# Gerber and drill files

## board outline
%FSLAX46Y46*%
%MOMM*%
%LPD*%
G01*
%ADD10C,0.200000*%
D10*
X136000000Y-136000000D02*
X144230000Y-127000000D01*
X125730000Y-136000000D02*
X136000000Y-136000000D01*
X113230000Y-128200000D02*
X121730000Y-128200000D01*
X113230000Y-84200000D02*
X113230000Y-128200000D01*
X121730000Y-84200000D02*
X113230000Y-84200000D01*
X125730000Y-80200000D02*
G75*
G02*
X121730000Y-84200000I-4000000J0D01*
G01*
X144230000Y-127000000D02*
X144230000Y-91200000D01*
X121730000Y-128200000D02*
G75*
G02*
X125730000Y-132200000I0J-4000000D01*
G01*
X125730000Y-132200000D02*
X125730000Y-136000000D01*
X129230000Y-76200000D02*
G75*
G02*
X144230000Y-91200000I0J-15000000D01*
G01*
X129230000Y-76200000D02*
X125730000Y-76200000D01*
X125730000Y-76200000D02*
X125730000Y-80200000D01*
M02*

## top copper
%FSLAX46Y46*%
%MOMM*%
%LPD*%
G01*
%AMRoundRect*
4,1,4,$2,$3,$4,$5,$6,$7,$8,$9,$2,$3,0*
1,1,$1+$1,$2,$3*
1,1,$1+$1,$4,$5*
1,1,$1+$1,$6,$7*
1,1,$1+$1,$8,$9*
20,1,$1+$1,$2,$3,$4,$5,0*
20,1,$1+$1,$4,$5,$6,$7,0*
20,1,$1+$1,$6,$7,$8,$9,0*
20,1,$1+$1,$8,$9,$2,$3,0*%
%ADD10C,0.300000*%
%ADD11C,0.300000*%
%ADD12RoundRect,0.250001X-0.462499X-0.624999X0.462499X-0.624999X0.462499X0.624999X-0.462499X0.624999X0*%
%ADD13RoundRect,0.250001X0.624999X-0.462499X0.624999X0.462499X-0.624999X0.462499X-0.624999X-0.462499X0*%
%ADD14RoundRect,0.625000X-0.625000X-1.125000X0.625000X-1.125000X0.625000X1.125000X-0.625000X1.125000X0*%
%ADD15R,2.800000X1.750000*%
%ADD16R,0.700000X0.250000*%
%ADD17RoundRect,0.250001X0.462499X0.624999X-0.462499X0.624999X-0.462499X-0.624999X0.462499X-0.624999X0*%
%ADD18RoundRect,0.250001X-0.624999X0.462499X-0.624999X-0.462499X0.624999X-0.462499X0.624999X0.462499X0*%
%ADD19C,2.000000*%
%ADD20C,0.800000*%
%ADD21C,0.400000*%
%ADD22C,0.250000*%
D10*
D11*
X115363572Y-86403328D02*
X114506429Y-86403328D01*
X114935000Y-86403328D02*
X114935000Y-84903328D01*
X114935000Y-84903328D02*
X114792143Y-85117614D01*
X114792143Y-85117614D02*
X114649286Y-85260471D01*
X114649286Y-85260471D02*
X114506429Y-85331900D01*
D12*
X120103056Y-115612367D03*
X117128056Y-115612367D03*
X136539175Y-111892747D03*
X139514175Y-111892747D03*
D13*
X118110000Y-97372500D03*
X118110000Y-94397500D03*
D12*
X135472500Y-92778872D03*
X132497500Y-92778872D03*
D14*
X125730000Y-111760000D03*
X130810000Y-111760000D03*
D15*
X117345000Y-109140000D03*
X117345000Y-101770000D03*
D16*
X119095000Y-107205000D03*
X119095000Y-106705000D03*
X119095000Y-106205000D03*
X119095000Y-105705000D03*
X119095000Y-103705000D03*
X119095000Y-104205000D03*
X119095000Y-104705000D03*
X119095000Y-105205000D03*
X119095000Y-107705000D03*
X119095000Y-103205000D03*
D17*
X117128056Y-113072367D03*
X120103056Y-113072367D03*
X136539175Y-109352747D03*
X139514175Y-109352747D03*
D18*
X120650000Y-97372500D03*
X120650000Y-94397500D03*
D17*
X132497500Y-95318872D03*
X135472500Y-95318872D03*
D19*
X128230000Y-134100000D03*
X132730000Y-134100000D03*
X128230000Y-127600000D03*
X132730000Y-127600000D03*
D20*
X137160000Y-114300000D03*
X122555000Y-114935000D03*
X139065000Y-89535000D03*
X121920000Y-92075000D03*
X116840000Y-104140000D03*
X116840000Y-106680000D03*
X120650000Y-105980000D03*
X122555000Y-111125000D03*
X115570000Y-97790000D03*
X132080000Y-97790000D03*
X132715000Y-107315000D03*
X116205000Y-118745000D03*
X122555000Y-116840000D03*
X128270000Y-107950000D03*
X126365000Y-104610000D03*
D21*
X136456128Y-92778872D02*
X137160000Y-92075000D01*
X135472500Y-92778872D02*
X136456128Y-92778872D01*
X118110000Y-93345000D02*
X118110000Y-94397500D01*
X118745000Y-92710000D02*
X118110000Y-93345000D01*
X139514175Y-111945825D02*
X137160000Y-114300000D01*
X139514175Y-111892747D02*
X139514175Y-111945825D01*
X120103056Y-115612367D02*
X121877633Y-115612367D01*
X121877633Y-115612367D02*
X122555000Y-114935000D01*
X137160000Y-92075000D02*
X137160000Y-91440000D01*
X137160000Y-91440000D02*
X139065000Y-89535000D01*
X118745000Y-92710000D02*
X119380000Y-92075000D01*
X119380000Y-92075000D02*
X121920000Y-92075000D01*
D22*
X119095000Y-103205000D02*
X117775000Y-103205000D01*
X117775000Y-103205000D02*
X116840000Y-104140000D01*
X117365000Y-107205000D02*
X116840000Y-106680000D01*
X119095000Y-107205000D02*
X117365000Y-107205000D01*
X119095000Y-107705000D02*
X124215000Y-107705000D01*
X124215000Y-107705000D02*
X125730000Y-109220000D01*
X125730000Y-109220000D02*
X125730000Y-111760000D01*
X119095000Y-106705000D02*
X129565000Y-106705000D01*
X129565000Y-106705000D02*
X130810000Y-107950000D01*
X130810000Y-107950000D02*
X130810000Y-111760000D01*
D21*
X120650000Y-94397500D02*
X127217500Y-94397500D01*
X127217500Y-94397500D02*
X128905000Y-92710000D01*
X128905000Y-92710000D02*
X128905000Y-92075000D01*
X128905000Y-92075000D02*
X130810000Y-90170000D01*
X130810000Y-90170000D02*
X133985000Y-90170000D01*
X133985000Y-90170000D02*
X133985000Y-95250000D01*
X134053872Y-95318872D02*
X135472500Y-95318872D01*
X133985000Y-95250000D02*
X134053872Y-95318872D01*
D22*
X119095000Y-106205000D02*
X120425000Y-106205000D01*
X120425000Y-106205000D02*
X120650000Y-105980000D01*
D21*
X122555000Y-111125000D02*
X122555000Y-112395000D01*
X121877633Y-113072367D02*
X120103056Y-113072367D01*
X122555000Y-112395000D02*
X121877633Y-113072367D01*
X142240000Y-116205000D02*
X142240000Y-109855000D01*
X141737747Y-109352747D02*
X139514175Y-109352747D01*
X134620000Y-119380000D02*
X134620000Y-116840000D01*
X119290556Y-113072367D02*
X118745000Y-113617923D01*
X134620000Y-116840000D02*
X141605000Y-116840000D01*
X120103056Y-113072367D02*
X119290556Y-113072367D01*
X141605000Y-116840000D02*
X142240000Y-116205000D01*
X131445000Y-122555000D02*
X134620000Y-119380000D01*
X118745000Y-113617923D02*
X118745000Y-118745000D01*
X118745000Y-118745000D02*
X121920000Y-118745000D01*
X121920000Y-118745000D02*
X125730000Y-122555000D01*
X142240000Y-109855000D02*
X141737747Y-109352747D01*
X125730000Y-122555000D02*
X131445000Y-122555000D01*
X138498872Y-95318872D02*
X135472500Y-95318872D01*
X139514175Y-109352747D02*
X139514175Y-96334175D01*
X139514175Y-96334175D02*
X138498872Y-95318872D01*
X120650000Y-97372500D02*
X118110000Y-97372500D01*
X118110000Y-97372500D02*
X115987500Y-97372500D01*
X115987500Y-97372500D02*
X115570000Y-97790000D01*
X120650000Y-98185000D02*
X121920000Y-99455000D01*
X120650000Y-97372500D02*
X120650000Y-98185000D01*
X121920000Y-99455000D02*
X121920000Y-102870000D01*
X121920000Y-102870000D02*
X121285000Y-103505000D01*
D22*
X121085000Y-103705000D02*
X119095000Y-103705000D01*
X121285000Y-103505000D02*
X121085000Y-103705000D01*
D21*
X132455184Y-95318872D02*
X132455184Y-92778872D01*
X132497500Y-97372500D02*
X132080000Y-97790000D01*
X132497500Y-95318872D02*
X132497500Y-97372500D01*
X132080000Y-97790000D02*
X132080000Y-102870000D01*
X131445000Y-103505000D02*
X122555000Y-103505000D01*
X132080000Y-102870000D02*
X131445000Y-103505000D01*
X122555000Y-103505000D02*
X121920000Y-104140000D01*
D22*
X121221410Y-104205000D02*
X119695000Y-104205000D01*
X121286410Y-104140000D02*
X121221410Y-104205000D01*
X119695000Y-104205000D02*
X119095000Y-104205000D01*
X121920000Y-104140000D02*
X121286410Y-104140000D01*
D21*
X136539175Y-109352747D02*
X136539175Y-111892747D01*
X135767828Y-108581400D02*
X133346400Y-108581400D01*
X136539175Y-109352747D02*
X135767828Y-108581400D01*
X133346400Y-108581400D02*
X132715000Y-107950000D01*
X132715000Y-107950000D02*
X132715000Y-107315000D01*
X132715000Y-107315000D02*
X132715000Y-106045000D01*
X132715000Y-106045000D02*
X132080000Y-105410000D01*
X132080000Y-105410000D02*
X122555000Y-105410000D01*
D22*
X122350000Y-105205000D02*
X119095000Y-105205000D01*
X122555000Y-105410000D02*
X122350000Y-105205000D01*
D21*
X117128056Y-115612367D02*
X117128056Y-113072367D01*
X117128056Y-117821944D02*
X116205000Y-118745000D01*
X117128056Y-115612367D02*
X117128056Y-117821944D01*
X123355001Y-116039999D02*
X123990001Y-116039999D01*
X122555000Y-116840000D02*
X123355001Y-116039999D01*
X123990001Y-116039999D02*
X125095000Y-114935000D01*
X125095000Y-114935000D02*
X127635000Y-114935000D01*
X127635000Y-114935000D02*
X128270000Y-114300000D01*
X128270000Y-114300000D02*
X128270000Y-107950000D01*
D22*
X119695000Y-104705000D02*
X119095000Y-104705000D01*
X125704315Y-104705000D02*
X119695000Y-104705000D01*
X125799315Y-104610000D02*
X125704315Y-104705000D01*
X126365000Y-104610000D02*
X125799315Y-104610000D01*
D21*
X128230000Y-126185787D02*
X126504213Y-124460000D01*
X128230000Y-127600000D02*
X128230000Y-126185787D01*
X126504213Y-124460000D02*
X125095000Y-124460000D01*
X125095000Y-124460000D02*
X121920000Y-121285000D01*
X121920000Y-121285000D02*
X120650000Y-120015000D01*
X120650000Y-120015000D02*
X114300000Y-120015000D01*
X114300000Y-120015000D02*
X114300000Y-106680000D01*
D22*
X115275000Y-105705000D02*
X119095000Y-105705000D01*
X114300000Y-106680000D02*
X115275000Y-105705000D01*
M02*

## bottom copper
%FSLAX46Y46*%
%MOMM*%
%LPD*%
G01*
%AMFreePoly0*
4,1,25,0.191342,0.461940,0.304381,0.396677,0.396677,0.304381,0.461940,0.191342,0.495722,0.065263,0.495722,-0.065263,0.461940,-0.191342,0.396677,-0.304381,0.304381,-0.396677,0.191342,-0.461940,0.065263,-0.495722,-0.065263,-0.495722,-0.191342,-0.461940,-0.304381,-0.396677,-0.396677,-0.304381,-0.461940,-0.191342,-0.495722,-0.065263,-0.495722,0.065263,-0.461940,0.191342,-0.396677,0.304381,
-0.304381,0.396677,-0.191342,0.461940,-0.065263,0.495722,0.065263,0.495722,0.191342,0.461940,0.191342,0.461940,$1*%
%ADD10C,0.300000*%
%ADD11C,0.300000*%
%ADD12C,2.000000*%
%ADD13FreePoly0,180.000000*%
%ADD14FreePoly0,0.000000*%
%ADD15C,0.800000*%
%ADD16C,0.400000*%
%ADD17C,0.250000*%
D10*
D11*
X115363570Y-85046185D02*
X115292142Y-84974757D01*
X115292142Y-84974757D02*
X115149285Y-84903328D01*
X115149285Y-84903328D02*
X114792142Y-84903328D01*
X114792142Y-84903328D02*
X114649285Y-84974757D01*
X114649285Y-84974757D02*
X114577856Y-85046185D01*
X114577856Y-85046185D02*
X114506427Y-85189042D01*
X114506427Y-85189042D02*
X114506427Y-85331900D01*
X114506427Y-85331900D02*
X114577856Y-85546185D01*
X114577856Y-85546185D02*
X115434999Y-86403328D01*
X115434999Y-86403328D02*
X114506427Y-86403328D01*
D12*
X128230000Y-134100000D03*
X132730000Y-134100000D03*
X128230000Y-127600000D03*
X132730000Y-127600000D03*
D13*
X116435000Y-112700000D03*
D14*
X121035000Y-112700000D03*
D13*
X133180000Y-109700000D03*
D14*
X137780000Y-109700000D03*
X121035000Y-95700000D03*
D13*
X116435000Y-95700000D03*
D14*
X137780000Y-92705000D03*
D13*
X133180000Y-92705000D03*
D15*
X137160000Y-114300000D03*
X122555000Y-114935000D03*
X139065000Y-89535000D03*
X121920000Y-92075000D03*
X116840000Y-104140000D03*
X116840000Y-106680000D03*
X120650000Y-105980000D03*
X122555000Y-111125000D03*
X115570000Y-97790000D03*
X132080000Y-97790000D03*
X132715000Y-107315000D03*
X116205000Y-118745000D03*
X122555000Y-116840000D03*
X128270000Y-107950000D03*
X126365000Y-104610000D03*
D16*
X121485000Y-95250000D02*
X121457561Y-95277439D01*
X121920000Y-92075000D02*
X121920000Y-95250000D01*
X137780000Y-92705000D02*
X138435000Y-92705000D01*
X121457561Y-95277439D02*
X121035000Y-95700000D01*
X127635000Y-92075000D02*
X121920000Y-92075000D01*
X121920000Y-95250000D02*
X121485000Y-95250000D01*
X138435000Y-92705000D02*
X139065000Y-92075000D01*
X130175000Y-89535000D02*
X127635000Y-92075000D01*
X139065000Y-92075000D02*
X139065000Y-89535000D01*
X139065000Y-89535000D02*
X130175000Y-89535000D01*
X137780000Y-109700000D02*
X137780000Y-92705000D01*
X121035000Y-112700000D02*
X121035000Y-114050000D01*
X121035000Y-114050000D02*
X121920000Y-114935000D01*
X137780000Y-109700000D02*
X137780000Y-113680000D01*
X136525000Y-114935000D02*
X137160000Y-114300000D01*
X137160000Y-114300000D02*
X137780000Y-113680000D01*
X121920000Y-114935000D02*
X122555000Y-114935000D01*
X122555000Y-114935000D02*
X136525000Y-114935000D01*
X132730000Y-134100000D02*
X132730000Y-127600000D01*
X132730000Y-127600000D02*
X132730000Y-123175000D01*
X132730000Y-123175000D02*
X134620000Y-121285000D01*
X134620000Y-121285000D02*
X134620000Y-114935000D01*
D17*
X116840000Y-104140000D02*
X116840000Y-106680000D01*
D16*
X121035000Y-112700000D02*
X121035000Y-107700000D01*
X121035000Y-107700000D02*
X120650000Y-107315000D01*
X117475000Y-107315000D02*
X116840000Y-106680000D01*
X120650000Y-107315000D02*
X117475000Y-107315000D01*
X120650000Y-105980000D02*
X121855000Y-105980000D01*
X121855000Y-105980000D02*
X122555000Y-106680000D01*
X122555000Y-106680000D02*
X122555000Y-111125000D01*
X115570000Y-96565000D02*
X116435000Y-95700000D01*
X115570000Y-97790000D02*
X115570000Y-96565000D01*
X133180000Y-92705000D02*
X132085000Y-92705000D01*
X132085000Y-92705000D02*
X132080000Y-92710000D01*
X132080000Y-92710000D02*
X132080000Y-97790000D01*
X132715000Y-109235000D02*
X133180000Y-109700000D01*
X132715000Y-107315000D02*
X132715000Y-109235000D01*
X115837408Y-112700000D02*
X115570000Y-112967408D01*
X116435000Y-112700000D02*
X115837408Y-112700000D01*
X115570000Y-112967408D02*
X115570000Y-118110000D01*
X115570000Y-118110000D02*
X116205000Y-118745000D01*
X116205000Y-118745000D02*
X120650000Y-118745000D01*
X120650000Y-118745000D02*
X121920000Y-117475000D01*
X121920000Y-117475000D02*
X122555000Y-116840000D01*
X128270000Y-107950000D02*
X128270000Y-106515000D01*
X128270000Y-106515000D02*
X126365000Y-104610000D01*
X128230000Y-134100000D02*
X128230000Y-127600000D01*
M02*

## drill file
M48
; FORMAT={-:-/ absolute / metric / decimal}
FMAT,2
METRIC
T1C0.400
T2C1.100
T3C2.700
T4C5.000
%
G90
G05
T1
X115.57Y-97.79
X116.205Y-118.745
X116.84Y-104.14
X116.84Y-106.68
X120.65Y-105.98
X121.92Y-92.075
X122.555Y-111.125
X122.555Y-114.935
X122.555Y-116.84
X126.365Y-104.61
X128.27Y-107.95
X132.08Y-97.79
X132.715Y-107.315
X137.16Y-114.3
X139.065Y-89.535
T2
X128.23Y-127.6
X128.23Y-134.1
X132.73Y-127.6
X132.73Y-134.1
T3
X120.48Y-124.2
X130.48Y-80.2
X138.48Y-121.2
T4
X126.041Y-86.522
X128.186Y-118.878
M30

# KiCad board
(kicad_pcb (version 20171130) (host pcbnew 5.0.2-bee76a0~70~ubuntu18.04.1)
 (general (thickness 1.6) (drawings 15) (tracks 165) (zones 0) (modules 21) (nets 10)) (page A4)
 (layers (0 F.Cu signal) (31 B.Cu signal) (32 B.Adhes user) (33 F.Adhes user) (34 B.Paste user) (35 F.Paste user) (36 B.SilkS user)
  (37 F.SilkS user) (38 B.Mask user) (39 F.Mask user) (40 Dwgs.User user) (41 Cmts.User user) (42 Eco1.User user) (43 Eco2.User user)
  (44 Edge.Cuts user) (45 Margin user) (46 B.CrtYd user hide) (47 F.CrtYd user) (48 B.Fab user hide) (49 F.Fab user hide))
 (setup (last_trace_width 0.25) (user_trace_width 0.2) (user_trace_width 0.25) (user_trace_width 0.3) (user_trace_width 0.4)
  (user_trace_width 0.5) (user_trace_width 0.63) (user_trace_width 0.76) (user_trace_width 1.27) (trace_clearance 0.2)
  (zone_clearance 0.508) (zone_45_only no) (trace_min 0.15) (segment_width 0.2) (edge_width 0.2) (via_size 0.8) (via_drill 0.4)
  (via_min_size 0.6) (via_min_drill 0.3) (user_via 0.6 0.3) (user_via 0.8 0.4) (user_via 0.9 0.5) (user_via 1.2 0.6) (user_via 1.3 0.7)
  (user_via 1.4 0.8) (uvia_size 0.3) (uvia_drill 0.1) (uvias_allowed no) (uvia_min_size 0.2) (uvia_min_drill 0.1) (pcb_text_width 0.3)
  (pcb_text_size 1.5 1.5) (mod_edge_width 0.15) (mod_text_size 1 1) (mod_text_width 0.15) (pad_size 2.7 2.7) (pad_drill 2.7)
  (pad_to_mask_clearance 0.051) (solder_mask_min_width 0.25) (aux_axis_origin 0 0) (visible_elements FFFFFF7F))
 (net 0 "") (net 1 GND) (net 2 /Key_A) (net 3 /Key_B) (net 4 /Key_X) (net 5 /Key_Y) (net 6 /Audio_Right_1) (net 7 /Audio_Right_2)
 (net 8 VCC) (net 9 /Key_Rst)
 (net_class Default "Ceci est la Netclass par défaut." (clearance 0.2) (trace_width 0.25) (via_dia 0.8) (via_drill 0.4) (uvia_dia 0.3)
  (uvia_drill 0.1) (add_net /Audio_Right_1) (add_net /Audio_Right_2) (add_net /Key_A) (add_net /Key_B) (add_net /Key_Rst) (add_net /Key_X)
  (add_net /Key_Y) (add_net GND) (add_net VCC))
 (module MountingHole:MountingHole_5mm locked (layer F.Cu) (at 126.041 86.522)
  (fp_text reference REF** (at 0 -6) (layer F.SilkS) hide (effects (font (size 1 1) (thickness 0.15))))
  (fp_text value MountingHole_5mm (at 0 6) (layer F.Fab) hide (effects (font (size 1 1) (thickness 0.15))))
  (pad "" np_thru_hole circle (at 0 0) (size 5 5) (drill 5) (layers *.Cu *.Mask)))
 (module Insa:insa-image (layer F.Cu) (at 130.81 101.6)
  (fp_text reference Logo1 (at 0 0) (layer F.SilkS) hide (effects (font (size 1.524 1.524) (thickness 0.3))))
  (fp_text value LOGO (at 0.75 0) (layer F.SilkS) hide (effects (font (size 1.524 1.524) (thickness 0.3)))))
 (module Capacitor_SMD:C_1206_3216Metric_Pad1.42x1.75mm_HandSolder (layer F.Cu) (at 118.615556 115.612367)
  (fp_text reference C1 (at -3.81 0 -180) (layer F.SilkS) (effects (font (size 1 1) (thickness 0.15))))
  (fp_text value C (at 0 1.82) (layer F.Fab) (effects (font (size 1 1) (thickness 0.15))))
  (pad 2 smd roundrect (at 1.4875 0) (size 1.425 1.75) (layers F.Cu F.Paste F.Mask) (roundrect_rratio 0.175439) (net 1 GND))
  (pad 1 smd roundrect (at -1.4875 0) (size 1.425 1.75) (layers F.Cu F.Paste F.Mask) (roundrect_rratio 0.175439) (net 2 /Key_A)))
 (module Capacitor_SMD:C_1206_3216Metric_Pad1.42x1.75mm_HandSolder (layer F.Cu) (at 138.026675 111.892747)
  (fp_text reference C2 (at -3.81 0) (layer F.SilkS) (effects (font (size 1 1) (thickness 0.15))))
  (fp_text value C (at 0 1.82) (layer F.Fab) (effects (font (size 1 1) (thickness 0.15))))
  (pad 1 smd roundrect (at -1.4875 0) (size 1.425 1.75) (layers F.Cu F.Paste F.Mask) (roundrect_rratio 0.175439) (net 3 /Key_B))
  (pad 2 smd roundrect (at 1.4875 0) (size 1.425 1.75) (layers F.Cu F.Paste F.Mask) (roundrect_rratio 0.175439) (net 1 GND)))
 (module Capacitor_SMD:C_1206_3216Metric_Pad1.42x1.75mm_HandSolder (layer F.Cu) (at 118.11 95.885 90)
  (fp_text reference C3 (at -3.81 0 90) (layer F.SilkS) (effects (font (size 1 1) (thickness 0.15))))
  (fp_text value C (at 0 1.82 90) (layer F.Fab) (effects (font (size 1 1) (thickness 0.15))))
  (pad 1 smd roundrect (at -1.4875 0 90) (size 1.425 1.75) (layers F.Cu F.Paste F.Mask) (roundrect_rratio 0.175439) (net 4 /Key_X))
  (pad 2 smd roundrect (at 1.4875 0 90) (size 1.425 1.75) (layers F.Cu F.Paste F.Mask) (roundrect_rratio 0.175439) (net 1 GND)))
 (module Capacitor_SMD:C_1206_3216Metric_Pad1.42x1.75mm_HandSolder (layer F.Cu) (at 133.985 92.778872)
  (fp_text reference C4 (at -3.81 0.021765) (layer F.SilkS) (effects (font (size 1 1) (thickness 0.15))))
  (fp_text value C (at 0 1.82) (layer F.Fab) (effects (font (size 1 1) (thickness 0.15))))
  (pad 2 smd roundrect (at 1.4875 0) (size 1.425 1.75) (layers F.Cu F.Paste F.Mask) (roundrect_rratio 0.175439) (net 1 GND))
  (pad 1 smd roundrect (at -1.4875 0) (size 1.425 1.75) (layers F.Cu F.Paste F.Mask) (roundrect_rratio 0.175439) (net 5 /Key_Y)))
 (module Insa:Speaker (layer F.Cu) (at 128.27 111.76)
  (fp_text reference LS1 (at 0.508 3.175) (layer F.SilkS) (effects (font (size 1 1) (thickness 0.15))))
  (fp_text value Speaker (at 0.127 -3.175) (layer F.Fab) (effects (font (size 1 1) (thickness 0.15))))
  (pad 1 smd roundrect (at -2.54 0) (size 2.5 3.5) (layers F.Cu F.Paste F.Mask) (roundrect_rratio 0.25) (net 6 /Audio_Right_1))
  (pad 2 smd roundrect (at 2.54 0) (size 2.5 3.5) (layers F.Cu F.Paste F.Mask) (roundrect_rratio 0.25) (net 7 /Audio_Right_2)))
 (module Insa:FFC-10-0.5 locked (layer F.Cu) (at 118.745 105.455 90)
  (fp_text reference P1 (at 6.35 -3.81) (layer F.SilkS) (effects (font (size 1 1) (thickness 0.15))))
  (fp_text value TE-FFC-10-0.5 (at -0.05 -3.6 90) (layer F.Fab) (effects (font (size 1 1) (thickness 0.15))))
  (pad A smd rect (at -3.685 -1.4 90) (size 1.75 2.8) (layers F.Cu F.Paste F.Mask))
  (pad B smd rect (at 3.685 -1.4 90) (size 1.75 2.8) (layers F.Cu F.Paste F.Mask))
  (pad 2 smd rect (at -1.75 0.35 90) (size 0.25 0.7) (layers F.Cu F.Paste F.Mask) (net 1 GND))
  (pad 3 smd rect (at -1.25 0.35 90) (size 0.25 0.7) (layers F.Cu F.Paste F.Mask) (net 7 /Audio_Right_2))
  (pad 4 smd rect (at -0.75 0.35 90) (size 0.25 0.7) (layers F.Cu F.Paste F.Mask) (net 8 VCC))
  (pad 5 smd rect (at -0.25 0.35 90) (size 0.25 0.7) (layers F.Cu F.Paste F.Mask) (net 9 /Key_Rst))
  (pad 9 smd rect (at 1.75 0.35 90) (size 0.25 0.7) (layers F.Cu F.Paste F.Mask) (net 4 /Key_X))
  (pad 8 smd rect (at 1.25 0.35 90) (size 0.25 0.7) (layers F.Cu F.Paste F.Mask) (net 5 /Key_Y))
  (pad 7 smd rect (at 0.75 0.35 90) (size 0.25 0.7) (layers F.Cu F.Paste F.Mask) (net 2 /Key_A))
  (pad 6 smd rect (at 0.25 0.35 90) (size 0.25 0.7) (layers F.Cu F.Paste F.Mask) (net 3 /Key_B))
  (pad 1 smd rect (at -2.25 0.35 90) (size 0.25 0.7) (layers F.Cu F.Paste F.Mask) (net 6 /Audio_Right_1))
  (pad 10 smd rect (at 2.25 0.35 90) (size 0.25 0.7) (layers F.Cu F.Paste F.Mask) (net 1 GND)))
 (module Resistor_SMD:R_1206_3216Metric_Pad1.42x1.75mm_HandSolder (layer F.Cu) (at 118.615556 113.072367 180)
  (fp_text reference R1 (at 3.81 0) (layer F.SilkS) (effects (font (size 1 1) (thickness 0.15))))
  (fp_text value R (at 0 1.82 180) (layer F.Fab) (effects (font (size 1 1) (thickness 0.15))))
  (pad 2 smd roundrect (at 1.4875 0 180) (size 1.425 1.75) (layers F.Cu F.Paste F.Mask) (roundrect_rratio 0.175439) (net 2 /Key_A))
  (pad 1 smd roundrect (at -1.4875 0 180) (size 1.425 1.75) (layers F.Cu F.Paste F.Mask) (roundrect_rratio 0.175439) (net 8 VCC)))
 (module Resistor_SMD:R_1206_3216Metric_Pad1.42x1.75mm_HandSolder (layer F.Cu) (at 138.026675 109.352747 180)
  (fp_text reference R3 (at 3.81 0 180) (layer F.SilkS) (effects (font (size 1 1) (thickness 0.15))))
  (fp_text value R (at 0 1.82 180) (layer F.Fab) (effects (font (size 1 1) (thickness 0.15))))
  (pad 2 smd roundrect (at 1.4875 0 180) (size 1.425 1.75) (layers F.Cu F.Paste F.Mask) (roundrect_rratio 0.175439) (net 3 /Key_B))
  (pad 1 smd roundrect (at -1.4875 0 180) (size 1.425 1.75) (layers F.Cu F.Paste F.Mask) (roundrect_rratio 0.175439) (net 8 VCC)))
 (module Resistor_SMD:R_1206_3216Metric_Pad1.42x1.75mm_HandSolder (layer F.Cu) (at 120.65 95.885 270)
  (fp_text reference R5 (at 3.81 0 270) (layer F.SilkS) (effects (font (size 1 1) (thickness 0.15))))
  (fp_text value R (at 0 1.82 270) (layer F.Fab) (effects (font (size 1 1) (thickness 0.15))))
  (pad 2 smd roundrect (at 1.4875 0 270) (size 1.425 1.75) (layers F.Cu F.Paste F.Mask) (roundrect_rratio 0.175439) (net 4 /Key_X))
  (pad 1 smd roundrect (at -1.4875 0 270) (size 1.425 1.75) (layers F.Cu F.Paste F.Mask) (roundrect_rratio 0.175439) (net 8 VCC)))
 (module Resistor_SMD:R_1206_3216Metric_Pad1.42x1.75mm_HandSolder (layer F.Cu) (at 133.985 95.318872 180)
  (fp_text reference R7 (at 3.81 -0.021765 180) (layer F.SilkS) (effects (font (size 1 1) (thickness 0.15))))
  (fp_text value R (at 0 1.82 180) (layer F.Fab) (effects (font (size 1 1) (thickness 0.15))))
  (pad 2 smd roundrect (at 1.4875 0 180) (size 1.425 1.75) (layers F.Cu F.Paste F.Mask) (roundrect_rratio 0.175439) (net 5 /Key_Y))
  (pad 1 smd roundrect (at -1.4875 0 180) (size 1.425 1.75) (layers F.Cu F.Paste F.Mask) (roundrect_rratio 0.175439) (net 8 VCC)))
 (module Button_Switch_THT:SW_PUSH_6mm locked (layer B.Cu) (at 132.73 134.1 90)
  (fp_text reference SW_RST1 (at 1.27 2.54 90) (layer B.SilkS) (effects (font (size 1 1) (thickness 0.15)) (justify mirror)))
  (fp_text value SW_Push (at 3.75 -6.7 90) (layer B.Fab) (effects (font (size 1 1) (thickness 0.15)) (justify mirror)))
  (pad 2 thru_hole circle (at 0 -4.5) (size 2 2) (drill 1.1) (layers *.Cu *.Mask) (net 9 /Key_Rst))
  (pad 1 thru_hole circle (at 0 0) (size 2 2) (drill 1.1) (layers *.Cu *.Mask) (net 1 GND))
  (pad 2 thru_hole circle (at 6.5 -4.5) (size 2 2) (drill 1.1) (layers *.Cu *.Mask) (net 9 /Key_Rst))
  (pad 1 thru_hole circle (at 6.5 0) (size 2 2) (drill 1.1) (layers *.Cu *.Mask) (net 1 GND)))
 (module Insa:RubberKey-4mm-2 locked (layer B.Cu) (at 118.735 112.7)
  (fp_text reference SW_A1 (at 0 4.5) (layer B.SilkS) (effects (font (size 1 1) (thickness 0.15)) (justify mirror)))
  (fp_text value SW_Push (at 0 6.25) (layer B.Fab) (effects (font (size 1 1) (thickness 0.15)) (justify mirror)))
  (pad 2 smd custom (at -2.3 0 180) (size 1 1) (layers B.Cu B.Paste B.Mask) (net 2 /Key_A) (zone_connect 0)
   (options (clearance outline) (anchor circle)) (primitives))
  (pad 1 smd custom (at 2.3 0) (size 1 1) (layers B.Cu B.Paste B.Mask) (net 1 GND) (zone_connect 0)
   (options (clearance outline) (anchor circle)) (primitives)))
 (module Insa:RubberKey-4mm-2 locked (layer B.Cu) (at 135.48 109.7)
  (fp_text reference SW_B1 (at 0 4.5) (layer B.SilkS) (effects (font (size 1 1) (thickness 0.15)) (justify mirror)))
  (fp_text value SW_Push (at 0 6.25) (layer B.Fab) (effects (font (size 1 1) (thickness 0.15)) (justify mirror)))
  (pad 2 smd custom (at -2.3 0 180) (size 1 1) (layers B.Cu B.Paste B.Mask) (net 3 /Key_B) (zone_connect 0)
   (options (clearance outline) (anchor circle)) (primitives))
  (pad 1 smd custom (at 2.3 0) (size 1 1) (layers B.Cu B.Paste B.Mask) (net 1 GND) (zone_connect 0)
   (options (clearance outline) (anchor circle)) (primitives)))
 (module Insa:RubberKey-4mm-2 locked (layer B.Cu) (at 118.735 95.7)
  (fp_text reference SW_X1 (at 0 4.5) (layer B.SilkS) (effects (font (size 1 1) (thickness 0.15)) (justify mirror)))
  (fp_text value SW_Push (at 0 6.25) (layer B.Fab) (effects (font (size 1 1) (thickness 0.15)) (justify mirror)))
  (pad 1 smd custom (at 2.3 0) (size 1 1) (layers B.Cu B.Paste B.Mask) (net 1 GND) (zone_connect 0)
   (options (clearance outline) (anchor circle)) (primitives))
  (pad 2 smd custom (at -2.3 0 180) (size 1 1) (layers B.Cu B.Paste B.Mask) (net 4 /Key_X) (zone_connect 0)
   (options (clearance outline) (anchor circle)) (primitives)))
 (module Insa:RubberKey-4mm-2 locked (layer B.Cu) (at 135.48 92.705)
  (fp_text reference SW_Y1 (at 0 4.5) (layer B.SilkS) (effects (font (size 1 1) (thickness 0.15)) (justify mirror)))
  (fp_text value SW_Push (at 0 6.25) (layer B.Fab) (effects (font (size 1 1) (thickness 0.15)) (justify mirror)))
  (pad 1 smd custom (at 2.3 0) (size 1 1) (layers B.Cu B.Paste B.Mask) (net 1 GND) (zone_connect 0)
   (options (clearance outline) (anchor circle)) (primitives))
  (pad 2 smd custom (at -2.3 0 180) (size 1 1) (layers B.Cu B.Paste B.Mask) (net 5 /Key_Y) (zone_connect 0)
   (options (clearance outline) (anchor circle)) (primitives)))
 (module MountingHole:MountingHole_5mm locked (layer F.Cu) (at 128.186 118.878)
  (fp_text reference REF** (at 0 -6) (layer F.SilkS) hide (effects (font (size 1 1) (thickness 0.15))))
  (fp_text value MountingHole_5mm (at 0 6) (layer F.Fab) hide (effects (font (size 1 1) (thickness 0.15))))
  (pad "" np_thru_hole circle (at 0 0) (size 5 5) (drill 5) (layers *.Cu *.Mask)))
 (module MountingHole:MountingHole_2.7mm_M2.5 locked (layer F.Cu) (at 138.48 121.2)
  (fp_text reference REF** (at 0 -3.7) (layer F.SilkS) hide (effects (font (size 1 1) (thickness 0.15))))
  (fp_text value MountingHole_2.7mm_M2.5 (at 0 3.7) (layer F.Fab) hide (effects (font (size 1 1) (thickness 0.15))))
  (pad "" np_thru_hole circle (at 0 0) (size 2.7 2.7) (drill 2.7) (layers *.Cu *.Mask)))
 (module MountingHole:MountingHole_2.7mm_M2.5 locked (layer F.Cu) (at 120.48 124.2)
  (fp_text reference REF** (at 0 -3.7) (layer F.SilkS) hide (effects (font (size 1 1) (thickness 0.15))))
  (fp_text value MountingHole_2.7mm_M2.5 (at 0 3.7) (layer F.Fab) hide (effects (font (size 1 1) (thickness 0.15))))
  (pad "" np_thru_hole circle (at 0 0) (size 2.7 2.7) (drill 2.7) (layers *.Cu *.Mask)))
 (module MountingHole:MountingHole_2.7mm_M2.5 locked (layer F.Cu) (at 130.48 80.2)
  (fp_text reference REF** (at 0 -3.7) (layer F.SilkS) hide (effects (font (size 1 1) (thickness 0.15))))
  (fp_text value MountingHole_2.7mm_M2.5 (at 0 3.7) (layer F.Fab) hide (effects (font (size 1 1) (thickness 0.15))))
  (pad "" np_thru_hole circle (at 0 0) (size 2.7 2.7) (drill 2.7) (layers *.Cu *.Mask)))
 (gr_line (start 136 136) (end 144.23 127) (layer Edge.Cuts) (width 0.2))
 (gr_line (start 125.73 136) (end 136 136) (layer Edge.Cuts) (width 0.2))
 (gr_line (start 113.23 128.2) (end 121.73 128.2) (layer Edge.Cuts) (width 0.2))
 (gr_line (start 113.23 84.2) (end 113.23 128.2) (layer Edge.Cuts) (width 0.2))
 (gr_line (start 121.73 84.2) (end 113.23 84.2) (layer Edge.Cuts) (width 0.2))
 (gr_arc (start 121.73 80.2) (end 121.73 84.2) (angle -90) (layer Edge.Cuts) (width 0.2))
 (gr_line (start 144.23 127) (end 144.23 91.2) (layer Edge.Cuts) (width 0.2))
 (gr_arc (start 121.73 132.2) (end 125.73 132.2) (angle -90) (layer Edge.Cuts) (width 0.2))
 (gr_line (start 125.73 132.2) (end 125.73 136) (layer Edge.Cuts) (width 0.2))
 (gr_arc (start 129.23 91.2) (end 144.23 91.2) (angle -90) (layer Edge.Cuts) (width 0.2))
 (gr_line (start 129.23 76.2) (end 125.73 76.2) (layer Edge.Cuts) (width 0.2))
 (gr_line (start 125.73 76.2) (end 125.73 80.2) (layer Edge.Cuts) (width 0.2))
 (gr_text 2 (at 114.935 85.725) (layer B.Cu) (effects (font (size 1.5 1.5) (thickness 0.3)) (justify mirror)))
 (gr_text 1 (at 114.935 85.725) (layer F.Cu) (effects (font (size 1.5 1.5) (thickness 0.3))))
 (segment (start 136.456128 92.778872) (end 137.16 92.075) (width 0.4) (layer F.Cu) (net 1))
 (segment (start 135.4725 92.778872) (end 136.456128 92.778872) (width 0.4) (layer F.Cu) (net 1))
 (segment (start 118.11 93.345) (end 118.11 94.3975) (width 0.4) (layer F.Cu) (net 1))
 (segment (start 118.745 92.71) (end 118.11 93.345) (width 0.4) (layer F.Cu) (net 1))
 (segment (start 121.485 95.25) (end 121.457561 95.277439) (width 0.4) (layer B.Cu) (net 1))
 (segment (start 121.92 92.075) (end 121.92 95.25) (width 0.4) (layer B.Cu) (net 1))
 (segment (start 137.78 92.705) (end 138.435 92.705) (width 0.4) (layer B.Cu) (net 1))
 (segment (start 121.457561 95.277439) (end 121.035 95.7) (width 0.4) (layer B.Cu) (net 1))
 (segment (start 127.635 92.075) (end 121.92 92.075) (width 0.4) (layer B.Cu) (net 1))
 (segment (start 121.92 95.25) (end 121.485 95.25) (width 0.4) (layer B.Cu) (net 1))
 (segment (start 138.435 92.705) (end 139.065 92.075) (width 0.4) (layer B.Cu) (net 1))
 (segment (start 130.175 89.535) (end 127.635 92.075) (width 0.4) (layer B.Cu) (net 1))
 (segment (start 139.065 92.075) (end 139.065 89.535) (width 0.4) (layer B.Cu) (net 1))
 (segment (start 139.065 89.535) (end 130.175 89.535) (width 0.4) (layer B.Cu) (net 1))
 (segment (start 137.78 109.7) (end 137.78 92.705) (width 0.4) (layer B.Cu) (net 1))
 (segment (start 121.035 112.7) (end 121.035 114.05) (width 0.4) (layer B.Cu) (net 1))
 (segment (start 121.035 114.05) (end 121.92 114.935) (width 0.4) (layer B.Cu) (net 1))
 (segment (start 137.78 109.7) (end 137.78 113.68) (width 0.4) (layer B.Cu) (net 1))
 (via (at 137.16 114.3) (size 0.8) (drill 0.4) (layers F.Cu B.Cu) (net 1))
 (segment (start 139.514175 111.945825) (end 137.16 114.3) (width 0.4) (layer F.Cu) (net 1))
 (segment (start 139.514175 111.892747) (end 139.514175 111.945825) (width 0.4) (layer F.Cu) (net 1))
 (segment (start 136.525 114.935) (end 137.16 114.3) (width 0.4) (layer B.Cu) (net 1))
 (segment (start 137.16 114.3) (end 137.78 113.68) (width 0.4) (layer B.Cu) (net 1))
 (segment (start 120.103056 115.612367) (end 121.877633 115.612367) (width 0.4) (layer F.Cu) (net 1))
 (via (at 122.555 114.935) (size 0.8) (drill 0.4) (layers F.Cu B.Cu) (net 1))
 (segment (start 121.877633 115.612367) (end 122.555 114.935) (width 0.4) (layer F.Cu) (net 1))
 (segment (start 121.92 114.935) (end 122.555 114.935) (width 0.4) (layer B.Cu) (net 1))
 (segment (start 122.555 114.935) (end 136.525 114.935) (width 0.4) (layer B.Cu) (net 1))
 (segment (start 132.73 134.1) (end 132.73 127.6) (width 0.4) (layer B.Cu) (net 1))
 (segment (start 132.73 127.6) (end 132.73 123.175) (width 0.4) (layer B.Cu) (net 1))
 (segment (start 132.73 123.175) (end 134.62 121.285) (width 0.4) (layer B.Cu) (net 1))
 (segment (start 134.62 121.285) (end 134.62 114.935) (width 0.4) (layer B.Cu) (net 1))
 (segment (start 137.16 92.075) (end 137.16 91.44) (width 0.4) (layer F.Cu) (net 1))
 (segment (start 137.16 91.44) (end 139.065 89.535) (width 0.4) (layer F.Cu) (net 1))
 (via (at 139.065 89.535) (size 0.8) (drill 0.4) (layers F.Cu B.Cu) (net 1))
 (segment (start 118.745 92.71) (end 119.38 92.075) (width 0.4) (layer F.Cu) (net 1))
 (segment (start 119.38 92.075) (end 121.92 92.075) (width 0.4) (layer F.Cu) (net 1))
 (via (at 121.92 92.075) (size 0.8) (drill 0.4) (layers F.Cu B.Cu) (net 1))
 (segment (start 119.095 103.205) (end 117.775 103.205) (width 0.25) (layer F.Cu) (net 1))
 (via (at 116.84 104.14) (size 0.8) (drill 0.4) (layers F.Cu B.Cu) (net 1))
 (segment (start 117.775 103.205) (end 116.84 104.14) (width 0.25) (layer F.Cu) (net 1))
 (segment (start 116.84 104.14) (end 116.84 106.68) (width 0.25) (layer B.Cu) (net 1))
 (via (at 116.84 106.68) (size 0.8) (drill 0.4) (layers F.Cu B.Cu) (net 1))
 (segment (start 117.365 107.205) (end 116.84 106.68) (width 0.25) (layer F.Cu) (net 1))
 (segment (start 119.095 107.205) (end 117.365 107.205) (width 0.25) (layer F.Cu) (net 1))
 (segment (start 121.035 112.7) (end 121.035 107.7) (width 0.4) (layer B.Cu) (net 1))
 (segment (start 121.035 107.7) (end 120.65 107.315) (width 0.4) (layer B.Cu) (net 1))
 (segment (start 117.475 107.315) (end 116.84 106.68) (width 0.4) (layer B.Cu) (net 1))
 (segment (start 120.65 107.315) (end 117.475 107.315) (width 0.4) (layer B.Cu) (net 1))
 (segment (start 119.095 107.705) (end 124.215 107.705) (width 0.25) (layer F.Cu) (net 6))
 (segment (start 124.215 107.705) (end 125.73 109.22) (width 0.25) (layer F.Cu) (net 6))
 (segment (start 125.73 109.22) (end 125.73 111.76) (width 0.25) (layer F.Cu) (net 6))
 (segment (start 119.095 106.705) (end 129.565 106.705) (width 0.25) (layer F.Cu) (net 7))
 (segment (start 129.565 106.705) (end 130.81 107.95) (width 0.25) (layer F.Cu) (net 7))
 (segment (start 130.81 107.95) (end 130.81 111.76) (width 0.25) (layer F.Cu) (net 7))
 (segment (start 120.65 94.3975) (end 127.2175 94.3975) (width 0.4) (layer F.Cu) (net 8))
 (segment (start 127.2175 94.3975) (end 128.905 92.71) (width 0.4) (layer F.Cu) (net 8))
 (segment (start 128.905 92.71) (end 128.905 92.075) (width 0.4) (layer F.Cu) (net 8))
 (segment (start 128.905 92.075) (end 130.81 90.17) (width 0.4) (layer F.Cu) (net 8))
 (segment (start 130.81 90.17) (end 133.985 90.17) (width 0.4) (layer F.Cu) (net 8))
 (segment (start 133.985 90.17) (end 133.985 95.25) (width 0.4) (layer F.Cu) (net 8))
 (segment (start 134.053872 95.318872) (end 135.4725 95.318872) (width 0.4) (layer F.Cu) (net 8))
 (segment (start 133.985 95.25) (end 134.053872 95.318872) (width 0.4) (layer F.Cu) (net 8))
 (via (at 120.65 105.98) (size 0.8) (drill 0.4) (layers F.Cu B.Cu) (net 8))
 (segment (start 119.095 106.205) (end 120.425 106.205) (width 0.25) (layer F.Cu) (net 8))
 (segment (start 120.425 106.205) (end 120.65 105.98) (width 0.25) (layer F.Cu) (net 8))
 (segment (start 120.65 105.98) (end 121.855 105.98) (width 0.4) (layer B.Cu) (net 8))
 (segment (start 121.855 105.98) (end 122.555 106.68) (width 0.4) (layer B.Cu) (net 8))
 (via (at 122.555 111.125) (size 0.8) (drill 0.4) (layers F.Cu B.Cu) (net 8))
 (segment (start 122.555 106.68) (end 122.555 111.125) (width 0.4) (layer B.Cu) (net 8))
 (segment (start 122.555 111.125) (end 122.555 112.395) (width 0.4) (layer F.Cu) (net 8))
 (segment (start 121.877633 113.072367) (end 120.103056 113.072367) (width 0.4) (layer F.Cu) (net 8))
 (segment (start 122.555 112.395) (end 121.877633 113.072367) (width 0.4) (layer F.Cu) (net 8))
 (segment (start 142.24 116.205) (end 142.24 109.855) (width 0.4) (layer F.Cu) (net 8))
 (segment (start 141.737747 109.352747) (end 139.514175 109.352747) (width 0.4) (layer F.Cu) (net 8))
 (segment (start 134.62 119.38) (end 134.62 116.84) (width 0.4) (layer F.Cu) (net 8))
 (segment (start 119.290556 113.072367) (end 118.745 113.617923) (width 0.4) (layer F.Cu) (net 8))
 (segment (start 134.62 116.84) (end 141.605 116.84) (width 0.4) (layer F.Cu) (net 8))
 (segment (start 120.103056 113.072367) (end 119.290556 113.072367) (width 0.4) (layer F.Cu) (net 8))
 (segment (start 141.605 116.84) (end 142.24 116.205) (width 0.4) (layer F.Cu) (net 8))
 (segment (start 131.445 122.555) (end 134.62 119.38) (width 0.4) (layer F.Cu) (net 8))
 (segment (start 118.745 113.617923) (end 118.745 118.745) (width 0.4) (layer F.Cu) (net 8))
 (segment (start 118.745 118.745) (end 121.92 118.745) (width 0.4) (layer F.Cu) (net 8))
 (segment (start 121.92 118.745) (end 125.73 122.555) (width 0.4) (layer F.Cu) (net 8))
 (segment (start 142.24 109.855) (end 141.737747 109.352747) (width 0.4) (layer F.Cu) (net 8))
 (segment (start 125.73 122.555) (end 131.445 122.555) (width 0.4) (layer F.Cu) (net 8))
 (segment (start 138.498872 95.318872) (end 135.4725 95.318872) (width 0.4) (layer F.Cu) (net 8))
 (segment (start 139.514175 109.352747) (end 139.514175 96.334175) (width 0.4) (layer F.Cu) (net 8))
 (segment (start 139.514175 96.334175) (end 138.498872 95.318872) (width 0.4) (layer F.Cu) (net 8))
 (segment (start 120.65 97.3725) (end 118.11 97.3725) (width 0.4) (layer F.Cu) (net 4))
 (segment (start 118.11 97.3725) (end 115.9875 97.3725) (width 0.4) (layer F.Cu) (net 4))
 (segment (start 115.9875 97.3725) (end 115.57 97.79) (width 0.4) (layer F.Cu) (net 4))
 (via (at 115.57 97.79) (size 0.8) (drill 0.4) (layers F.Cu B.Cu) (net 4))
 (segment (start 115.57 96.565) (end 116.435 95.7) (width 0.4) (layer B.Cu) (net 4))
 (segment (start 115.57 97.79) (end 115.57 96.565) (width 0.4) (layer B.Cu) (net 4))
 (segment (start 120.65 98.185) (end 121.92 99.455) (width 0.4) (layer F.Cu) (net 4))
 (segment (start 120.65 97.3725) (end 120.65 98.185) (width 0.4) (layer F.Cu) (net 4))
 (segment (start 121.92 99.455) (end 121.92 102.87) (width 0.4) (layer F.Cu) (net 4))
 (segment (start 121.92 102.87) (end 121.285 103.505) (width 0.4) (layer F.Cu) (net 4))
 (segment (start 121.085 103.705) (end 119.095 103.705) (width 0.25) (layer F.Cu) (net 4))
 (segment (start 121.285 103.505) (end 121.085 103.705) (width 0.25) (layer F.Cu) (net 4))
 (segment (start 132.455184 95.318872) (end 132.455184 92.778872) (width 0.4) (layer F.Cu) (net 5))
 (segment (start 133.18 92.705) (end 132.085 92.705) (width 0.4) (layer B.Cu) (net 5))
 (segment (start 132.085 92.705) (end 132.08 92.71) (width 0.4) (layer B.Cu) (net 5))
 (segment (start 132.08 92.71) (end 132.08 97.79) (width 0.4) (layer B.Cu) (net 5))
 (via (at 132.08 97.79) (size 0.8) (drill 0.4) (layers F.Cu B.Cu) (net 5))
 (segment (start 132.4975 97.3725) (end 132.08 97.79) (width 0.4) (layer F.Cu) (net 5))
 (segment (start 132.4975 95.318872) (end 132.4975 97.3725) (width 0.4) (layer F.Cu) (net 5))
 (segment (start 132.08 97.79) (end 132.08 102.87) (width 0.4) (layer F.Cu) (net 5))
 (segment (start 131.445 103.505) (end 122.555 103.505) (width 0.4) (layer F.Cu) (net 5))
 (segment (start 132.08 102.87) (end 131.445 103.505) (width 0.4) (layer F.Cu) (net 5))
 (segment (start 122.555 103.505) (end 121.92 104.14) (width 0.4) (layer F.Cu) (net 5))
 (segment (start 121.22141 104.205) (end 119.695 104.205) (width 0.25) (layer F.Cu) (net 5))
 (segment (start 121.28641 104.14) (end 121.22141 104.205) (width 0.25) (layer F.Cu) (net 5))
 (segment (start 119.695 104.205) (end 119.095 104.205) (width 0.25) (layer F.Cu) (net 5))
 (segment (start 121.92 104.14) (end 121.28641 104.14) (width 0.25) (layer F.Cu) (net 5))
 (segment (start 136.539175 109.352747) (end 136.539175 111.892747) (width 0.4) (layer F.Cu) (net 3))
 (segment (start 135.767828 108.5814) (end 133.3464 108.5814) (width 0.4) (layer F.Cu) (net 3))
 (segment (start 136.539175 109.352747) (end 135.767828 108.5814) (width 0.4) (layer F.Cu) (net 3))
 (segment (start 133.3464 108.5814) (end 132.715 107.95) (width 0.4) (layer F.Cu) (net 3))
 (via (at 132.715 107.315) (size 0.8) (drill 0.4) (layers F.Cu B.Cu) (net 3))
 (segment (start 132.715 107.95) (end 132.715 107.315) (width 0.4) (layer F.Cu) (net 3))
 (segment (start 132.715 109.235) (end 133.18 109.7) (width 0.4) (layer B.Cu) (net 3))
 (segment (start 132.715 107.315) (end 132.715 109.235) (width 0.4) (layer B.Cu) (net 3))
 (segment (start 132.715 107.315) (end 132.715 106.045) (width 0.4) (layer F.Cu) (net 3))
 (segment (start 132.715 106.045) (end 132.08 105.41) (width 0.4) (layer F.Cu) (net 3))
 (segment (start 132.08 105.41) (end 122.555 105.41) (width 0.4) (layer F.Cu) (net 3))
 (segment (start 122.35 105.205) (end 119.095 105.205) (width 0.25) (layer F.Cu) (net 3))
 (segment (start 122.555 105.41) (end 122.35 105.205) (width 0.25) (layer F.Cu) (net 3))
 (segment (start 117.128056 115.612367) (end 117.128056 113.072367) (width 0.4) (layer F.Cu) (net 2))
 (segment (start 115.837408 112.7) (end 115.57 112.967408) (width 0.4) (layer B.Cu) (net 2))
 (segment (start 116.435 112.7) (end 115.837408 112.7) (width 0.4) (layer B.Cu) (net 2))
 (segment (start 115.57 112.967408) (end 115.57 118.11) (width 0.4) (layer B.Cu) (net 2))
 (segment (start 115.57 118.11) (end 116.205 118.745) (width 0.4) (layer B.Cu) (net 2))
 (via (at 116.205 118.745) (size 0.8) (drill 0.4) (layers F.Cu B.Cu) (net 2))
 (segment (start 117.128056 117.821944) (end 116.205 118.745) (width 0.4) (layer F.Cu) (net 2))
 (segment (start 117.128056 115.612367) (end 117.128056 117.821944) (width 0.4) (layer F.Cu) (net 2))
 (segment (start 116.205 118.745) (end 120.65 118.745) (width 0.4) (layer B.Cu) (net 2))
 (segment (start 120.65 118.745) (end 121.92 117.475) (width 0.4) (layer B.Cu) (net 2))
 (via (at 122.555 116.84) (size 0.8) (drill 0.4) (layers F.Cu B.Cu) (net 2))
 (segment (start 121.92 117.475) (end 122.555 116.84) (width 0.4) (layer B.Cu) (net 2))
 (segment (start 123.355001 116.039999) (end 123.990001 116.039999) (width 0.4) (layer F.Cu) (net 2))
 (segment (start 122.555 116.84) (end 123.355001 116.039999) (width 0.4) (layer F.Cu) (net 2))
 (segment (start 123.990001 116.039999) (end 125.095 114.935) (width 0.4) (layer F.Cu) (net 2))
 (segment (start 125.095 114.935) (end 127.635 114.935) (width 0.4) (layer F.Cu) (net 2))
 (via (at 128.27 107.95) (size 0.8) (drill 0.4) (layers F.Cu B.Cu) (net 2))
 (segment (start 127.635 114.935) (end 128.27 114.3) (width 0.4) (layer F.Cu) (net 2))
 (segment (start 128.27 114.3) (end 128.27 107.95) (width 0.4) (layer F.Cu) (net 2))
 (via (at 126.365 104.61) (size 0.8) (drill 0.4) (layers F.Cu B.Cu) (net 2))
 (segment (start 128.27 107.95) (end 128.27 106.515) (width 0.4) (layer B.Cu) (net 2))
 (segment (start 128.27 106.515) (end 126.365 104.61) (width 0.4) (layer B.Cu) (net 2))
 (segment (start 119.695 104.705) (end 119.095 104.705) (width 0.25) (layer F.Cu) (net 2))
 (segment (start 125.704315 104.705) (end 119.695 104.705) (width 0.25) (layer F.Cu) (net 2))
 (segment (start 125.799315 104.61) (end 125.704315 104.705) (width 0.25) (layer F.Cu) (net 2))
 (segment (start 126.365 104.61) (end 125.799315 104.61) (width 0.25) (layer F.Cu) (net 2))
 (segment (start 128.23 134.1) (end 128.23 127.6) (width 0.4) (layer B.Cu) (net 9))
 (segment (start 128.23 126.185787) (end 126.504213 124.46) (width 0.4) (layer F.Cu) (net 9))
 (segment (start 128.23 127.6) (end 128.23 126.185787) (width 0.4) (layer F.Cu) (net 9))
 (segment (start 126.504213 124.46) (end 125.095 124.46) (width 0.4) (layer F.Cu) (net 9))
 (segment (start 125.095 124.46) (end 121.92 121.285) (width 0.4) (layer F.Cu) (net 9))
 (segment (start 121.92 121.285) (end 120.65 120.015) (width 0.4) (layer F.Cu) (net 9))
 (segment (start 120.65 120.015) (end 114.3 120.015) (width 0.4) (layer F.Cu) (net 9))
 (segment (start 114.3 120.015) (end 114.3 106.68) (width 0.4) (layer F.Cu) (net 9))
 (segment (start 115.275 105.705) (end 119.095 105.705) (width 0.25) (layer F.Cu) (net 9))
 (segment (start 114.3 106.68) (end 115.275 105.705) (width 0.25) (layer F.Cu) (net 9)))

